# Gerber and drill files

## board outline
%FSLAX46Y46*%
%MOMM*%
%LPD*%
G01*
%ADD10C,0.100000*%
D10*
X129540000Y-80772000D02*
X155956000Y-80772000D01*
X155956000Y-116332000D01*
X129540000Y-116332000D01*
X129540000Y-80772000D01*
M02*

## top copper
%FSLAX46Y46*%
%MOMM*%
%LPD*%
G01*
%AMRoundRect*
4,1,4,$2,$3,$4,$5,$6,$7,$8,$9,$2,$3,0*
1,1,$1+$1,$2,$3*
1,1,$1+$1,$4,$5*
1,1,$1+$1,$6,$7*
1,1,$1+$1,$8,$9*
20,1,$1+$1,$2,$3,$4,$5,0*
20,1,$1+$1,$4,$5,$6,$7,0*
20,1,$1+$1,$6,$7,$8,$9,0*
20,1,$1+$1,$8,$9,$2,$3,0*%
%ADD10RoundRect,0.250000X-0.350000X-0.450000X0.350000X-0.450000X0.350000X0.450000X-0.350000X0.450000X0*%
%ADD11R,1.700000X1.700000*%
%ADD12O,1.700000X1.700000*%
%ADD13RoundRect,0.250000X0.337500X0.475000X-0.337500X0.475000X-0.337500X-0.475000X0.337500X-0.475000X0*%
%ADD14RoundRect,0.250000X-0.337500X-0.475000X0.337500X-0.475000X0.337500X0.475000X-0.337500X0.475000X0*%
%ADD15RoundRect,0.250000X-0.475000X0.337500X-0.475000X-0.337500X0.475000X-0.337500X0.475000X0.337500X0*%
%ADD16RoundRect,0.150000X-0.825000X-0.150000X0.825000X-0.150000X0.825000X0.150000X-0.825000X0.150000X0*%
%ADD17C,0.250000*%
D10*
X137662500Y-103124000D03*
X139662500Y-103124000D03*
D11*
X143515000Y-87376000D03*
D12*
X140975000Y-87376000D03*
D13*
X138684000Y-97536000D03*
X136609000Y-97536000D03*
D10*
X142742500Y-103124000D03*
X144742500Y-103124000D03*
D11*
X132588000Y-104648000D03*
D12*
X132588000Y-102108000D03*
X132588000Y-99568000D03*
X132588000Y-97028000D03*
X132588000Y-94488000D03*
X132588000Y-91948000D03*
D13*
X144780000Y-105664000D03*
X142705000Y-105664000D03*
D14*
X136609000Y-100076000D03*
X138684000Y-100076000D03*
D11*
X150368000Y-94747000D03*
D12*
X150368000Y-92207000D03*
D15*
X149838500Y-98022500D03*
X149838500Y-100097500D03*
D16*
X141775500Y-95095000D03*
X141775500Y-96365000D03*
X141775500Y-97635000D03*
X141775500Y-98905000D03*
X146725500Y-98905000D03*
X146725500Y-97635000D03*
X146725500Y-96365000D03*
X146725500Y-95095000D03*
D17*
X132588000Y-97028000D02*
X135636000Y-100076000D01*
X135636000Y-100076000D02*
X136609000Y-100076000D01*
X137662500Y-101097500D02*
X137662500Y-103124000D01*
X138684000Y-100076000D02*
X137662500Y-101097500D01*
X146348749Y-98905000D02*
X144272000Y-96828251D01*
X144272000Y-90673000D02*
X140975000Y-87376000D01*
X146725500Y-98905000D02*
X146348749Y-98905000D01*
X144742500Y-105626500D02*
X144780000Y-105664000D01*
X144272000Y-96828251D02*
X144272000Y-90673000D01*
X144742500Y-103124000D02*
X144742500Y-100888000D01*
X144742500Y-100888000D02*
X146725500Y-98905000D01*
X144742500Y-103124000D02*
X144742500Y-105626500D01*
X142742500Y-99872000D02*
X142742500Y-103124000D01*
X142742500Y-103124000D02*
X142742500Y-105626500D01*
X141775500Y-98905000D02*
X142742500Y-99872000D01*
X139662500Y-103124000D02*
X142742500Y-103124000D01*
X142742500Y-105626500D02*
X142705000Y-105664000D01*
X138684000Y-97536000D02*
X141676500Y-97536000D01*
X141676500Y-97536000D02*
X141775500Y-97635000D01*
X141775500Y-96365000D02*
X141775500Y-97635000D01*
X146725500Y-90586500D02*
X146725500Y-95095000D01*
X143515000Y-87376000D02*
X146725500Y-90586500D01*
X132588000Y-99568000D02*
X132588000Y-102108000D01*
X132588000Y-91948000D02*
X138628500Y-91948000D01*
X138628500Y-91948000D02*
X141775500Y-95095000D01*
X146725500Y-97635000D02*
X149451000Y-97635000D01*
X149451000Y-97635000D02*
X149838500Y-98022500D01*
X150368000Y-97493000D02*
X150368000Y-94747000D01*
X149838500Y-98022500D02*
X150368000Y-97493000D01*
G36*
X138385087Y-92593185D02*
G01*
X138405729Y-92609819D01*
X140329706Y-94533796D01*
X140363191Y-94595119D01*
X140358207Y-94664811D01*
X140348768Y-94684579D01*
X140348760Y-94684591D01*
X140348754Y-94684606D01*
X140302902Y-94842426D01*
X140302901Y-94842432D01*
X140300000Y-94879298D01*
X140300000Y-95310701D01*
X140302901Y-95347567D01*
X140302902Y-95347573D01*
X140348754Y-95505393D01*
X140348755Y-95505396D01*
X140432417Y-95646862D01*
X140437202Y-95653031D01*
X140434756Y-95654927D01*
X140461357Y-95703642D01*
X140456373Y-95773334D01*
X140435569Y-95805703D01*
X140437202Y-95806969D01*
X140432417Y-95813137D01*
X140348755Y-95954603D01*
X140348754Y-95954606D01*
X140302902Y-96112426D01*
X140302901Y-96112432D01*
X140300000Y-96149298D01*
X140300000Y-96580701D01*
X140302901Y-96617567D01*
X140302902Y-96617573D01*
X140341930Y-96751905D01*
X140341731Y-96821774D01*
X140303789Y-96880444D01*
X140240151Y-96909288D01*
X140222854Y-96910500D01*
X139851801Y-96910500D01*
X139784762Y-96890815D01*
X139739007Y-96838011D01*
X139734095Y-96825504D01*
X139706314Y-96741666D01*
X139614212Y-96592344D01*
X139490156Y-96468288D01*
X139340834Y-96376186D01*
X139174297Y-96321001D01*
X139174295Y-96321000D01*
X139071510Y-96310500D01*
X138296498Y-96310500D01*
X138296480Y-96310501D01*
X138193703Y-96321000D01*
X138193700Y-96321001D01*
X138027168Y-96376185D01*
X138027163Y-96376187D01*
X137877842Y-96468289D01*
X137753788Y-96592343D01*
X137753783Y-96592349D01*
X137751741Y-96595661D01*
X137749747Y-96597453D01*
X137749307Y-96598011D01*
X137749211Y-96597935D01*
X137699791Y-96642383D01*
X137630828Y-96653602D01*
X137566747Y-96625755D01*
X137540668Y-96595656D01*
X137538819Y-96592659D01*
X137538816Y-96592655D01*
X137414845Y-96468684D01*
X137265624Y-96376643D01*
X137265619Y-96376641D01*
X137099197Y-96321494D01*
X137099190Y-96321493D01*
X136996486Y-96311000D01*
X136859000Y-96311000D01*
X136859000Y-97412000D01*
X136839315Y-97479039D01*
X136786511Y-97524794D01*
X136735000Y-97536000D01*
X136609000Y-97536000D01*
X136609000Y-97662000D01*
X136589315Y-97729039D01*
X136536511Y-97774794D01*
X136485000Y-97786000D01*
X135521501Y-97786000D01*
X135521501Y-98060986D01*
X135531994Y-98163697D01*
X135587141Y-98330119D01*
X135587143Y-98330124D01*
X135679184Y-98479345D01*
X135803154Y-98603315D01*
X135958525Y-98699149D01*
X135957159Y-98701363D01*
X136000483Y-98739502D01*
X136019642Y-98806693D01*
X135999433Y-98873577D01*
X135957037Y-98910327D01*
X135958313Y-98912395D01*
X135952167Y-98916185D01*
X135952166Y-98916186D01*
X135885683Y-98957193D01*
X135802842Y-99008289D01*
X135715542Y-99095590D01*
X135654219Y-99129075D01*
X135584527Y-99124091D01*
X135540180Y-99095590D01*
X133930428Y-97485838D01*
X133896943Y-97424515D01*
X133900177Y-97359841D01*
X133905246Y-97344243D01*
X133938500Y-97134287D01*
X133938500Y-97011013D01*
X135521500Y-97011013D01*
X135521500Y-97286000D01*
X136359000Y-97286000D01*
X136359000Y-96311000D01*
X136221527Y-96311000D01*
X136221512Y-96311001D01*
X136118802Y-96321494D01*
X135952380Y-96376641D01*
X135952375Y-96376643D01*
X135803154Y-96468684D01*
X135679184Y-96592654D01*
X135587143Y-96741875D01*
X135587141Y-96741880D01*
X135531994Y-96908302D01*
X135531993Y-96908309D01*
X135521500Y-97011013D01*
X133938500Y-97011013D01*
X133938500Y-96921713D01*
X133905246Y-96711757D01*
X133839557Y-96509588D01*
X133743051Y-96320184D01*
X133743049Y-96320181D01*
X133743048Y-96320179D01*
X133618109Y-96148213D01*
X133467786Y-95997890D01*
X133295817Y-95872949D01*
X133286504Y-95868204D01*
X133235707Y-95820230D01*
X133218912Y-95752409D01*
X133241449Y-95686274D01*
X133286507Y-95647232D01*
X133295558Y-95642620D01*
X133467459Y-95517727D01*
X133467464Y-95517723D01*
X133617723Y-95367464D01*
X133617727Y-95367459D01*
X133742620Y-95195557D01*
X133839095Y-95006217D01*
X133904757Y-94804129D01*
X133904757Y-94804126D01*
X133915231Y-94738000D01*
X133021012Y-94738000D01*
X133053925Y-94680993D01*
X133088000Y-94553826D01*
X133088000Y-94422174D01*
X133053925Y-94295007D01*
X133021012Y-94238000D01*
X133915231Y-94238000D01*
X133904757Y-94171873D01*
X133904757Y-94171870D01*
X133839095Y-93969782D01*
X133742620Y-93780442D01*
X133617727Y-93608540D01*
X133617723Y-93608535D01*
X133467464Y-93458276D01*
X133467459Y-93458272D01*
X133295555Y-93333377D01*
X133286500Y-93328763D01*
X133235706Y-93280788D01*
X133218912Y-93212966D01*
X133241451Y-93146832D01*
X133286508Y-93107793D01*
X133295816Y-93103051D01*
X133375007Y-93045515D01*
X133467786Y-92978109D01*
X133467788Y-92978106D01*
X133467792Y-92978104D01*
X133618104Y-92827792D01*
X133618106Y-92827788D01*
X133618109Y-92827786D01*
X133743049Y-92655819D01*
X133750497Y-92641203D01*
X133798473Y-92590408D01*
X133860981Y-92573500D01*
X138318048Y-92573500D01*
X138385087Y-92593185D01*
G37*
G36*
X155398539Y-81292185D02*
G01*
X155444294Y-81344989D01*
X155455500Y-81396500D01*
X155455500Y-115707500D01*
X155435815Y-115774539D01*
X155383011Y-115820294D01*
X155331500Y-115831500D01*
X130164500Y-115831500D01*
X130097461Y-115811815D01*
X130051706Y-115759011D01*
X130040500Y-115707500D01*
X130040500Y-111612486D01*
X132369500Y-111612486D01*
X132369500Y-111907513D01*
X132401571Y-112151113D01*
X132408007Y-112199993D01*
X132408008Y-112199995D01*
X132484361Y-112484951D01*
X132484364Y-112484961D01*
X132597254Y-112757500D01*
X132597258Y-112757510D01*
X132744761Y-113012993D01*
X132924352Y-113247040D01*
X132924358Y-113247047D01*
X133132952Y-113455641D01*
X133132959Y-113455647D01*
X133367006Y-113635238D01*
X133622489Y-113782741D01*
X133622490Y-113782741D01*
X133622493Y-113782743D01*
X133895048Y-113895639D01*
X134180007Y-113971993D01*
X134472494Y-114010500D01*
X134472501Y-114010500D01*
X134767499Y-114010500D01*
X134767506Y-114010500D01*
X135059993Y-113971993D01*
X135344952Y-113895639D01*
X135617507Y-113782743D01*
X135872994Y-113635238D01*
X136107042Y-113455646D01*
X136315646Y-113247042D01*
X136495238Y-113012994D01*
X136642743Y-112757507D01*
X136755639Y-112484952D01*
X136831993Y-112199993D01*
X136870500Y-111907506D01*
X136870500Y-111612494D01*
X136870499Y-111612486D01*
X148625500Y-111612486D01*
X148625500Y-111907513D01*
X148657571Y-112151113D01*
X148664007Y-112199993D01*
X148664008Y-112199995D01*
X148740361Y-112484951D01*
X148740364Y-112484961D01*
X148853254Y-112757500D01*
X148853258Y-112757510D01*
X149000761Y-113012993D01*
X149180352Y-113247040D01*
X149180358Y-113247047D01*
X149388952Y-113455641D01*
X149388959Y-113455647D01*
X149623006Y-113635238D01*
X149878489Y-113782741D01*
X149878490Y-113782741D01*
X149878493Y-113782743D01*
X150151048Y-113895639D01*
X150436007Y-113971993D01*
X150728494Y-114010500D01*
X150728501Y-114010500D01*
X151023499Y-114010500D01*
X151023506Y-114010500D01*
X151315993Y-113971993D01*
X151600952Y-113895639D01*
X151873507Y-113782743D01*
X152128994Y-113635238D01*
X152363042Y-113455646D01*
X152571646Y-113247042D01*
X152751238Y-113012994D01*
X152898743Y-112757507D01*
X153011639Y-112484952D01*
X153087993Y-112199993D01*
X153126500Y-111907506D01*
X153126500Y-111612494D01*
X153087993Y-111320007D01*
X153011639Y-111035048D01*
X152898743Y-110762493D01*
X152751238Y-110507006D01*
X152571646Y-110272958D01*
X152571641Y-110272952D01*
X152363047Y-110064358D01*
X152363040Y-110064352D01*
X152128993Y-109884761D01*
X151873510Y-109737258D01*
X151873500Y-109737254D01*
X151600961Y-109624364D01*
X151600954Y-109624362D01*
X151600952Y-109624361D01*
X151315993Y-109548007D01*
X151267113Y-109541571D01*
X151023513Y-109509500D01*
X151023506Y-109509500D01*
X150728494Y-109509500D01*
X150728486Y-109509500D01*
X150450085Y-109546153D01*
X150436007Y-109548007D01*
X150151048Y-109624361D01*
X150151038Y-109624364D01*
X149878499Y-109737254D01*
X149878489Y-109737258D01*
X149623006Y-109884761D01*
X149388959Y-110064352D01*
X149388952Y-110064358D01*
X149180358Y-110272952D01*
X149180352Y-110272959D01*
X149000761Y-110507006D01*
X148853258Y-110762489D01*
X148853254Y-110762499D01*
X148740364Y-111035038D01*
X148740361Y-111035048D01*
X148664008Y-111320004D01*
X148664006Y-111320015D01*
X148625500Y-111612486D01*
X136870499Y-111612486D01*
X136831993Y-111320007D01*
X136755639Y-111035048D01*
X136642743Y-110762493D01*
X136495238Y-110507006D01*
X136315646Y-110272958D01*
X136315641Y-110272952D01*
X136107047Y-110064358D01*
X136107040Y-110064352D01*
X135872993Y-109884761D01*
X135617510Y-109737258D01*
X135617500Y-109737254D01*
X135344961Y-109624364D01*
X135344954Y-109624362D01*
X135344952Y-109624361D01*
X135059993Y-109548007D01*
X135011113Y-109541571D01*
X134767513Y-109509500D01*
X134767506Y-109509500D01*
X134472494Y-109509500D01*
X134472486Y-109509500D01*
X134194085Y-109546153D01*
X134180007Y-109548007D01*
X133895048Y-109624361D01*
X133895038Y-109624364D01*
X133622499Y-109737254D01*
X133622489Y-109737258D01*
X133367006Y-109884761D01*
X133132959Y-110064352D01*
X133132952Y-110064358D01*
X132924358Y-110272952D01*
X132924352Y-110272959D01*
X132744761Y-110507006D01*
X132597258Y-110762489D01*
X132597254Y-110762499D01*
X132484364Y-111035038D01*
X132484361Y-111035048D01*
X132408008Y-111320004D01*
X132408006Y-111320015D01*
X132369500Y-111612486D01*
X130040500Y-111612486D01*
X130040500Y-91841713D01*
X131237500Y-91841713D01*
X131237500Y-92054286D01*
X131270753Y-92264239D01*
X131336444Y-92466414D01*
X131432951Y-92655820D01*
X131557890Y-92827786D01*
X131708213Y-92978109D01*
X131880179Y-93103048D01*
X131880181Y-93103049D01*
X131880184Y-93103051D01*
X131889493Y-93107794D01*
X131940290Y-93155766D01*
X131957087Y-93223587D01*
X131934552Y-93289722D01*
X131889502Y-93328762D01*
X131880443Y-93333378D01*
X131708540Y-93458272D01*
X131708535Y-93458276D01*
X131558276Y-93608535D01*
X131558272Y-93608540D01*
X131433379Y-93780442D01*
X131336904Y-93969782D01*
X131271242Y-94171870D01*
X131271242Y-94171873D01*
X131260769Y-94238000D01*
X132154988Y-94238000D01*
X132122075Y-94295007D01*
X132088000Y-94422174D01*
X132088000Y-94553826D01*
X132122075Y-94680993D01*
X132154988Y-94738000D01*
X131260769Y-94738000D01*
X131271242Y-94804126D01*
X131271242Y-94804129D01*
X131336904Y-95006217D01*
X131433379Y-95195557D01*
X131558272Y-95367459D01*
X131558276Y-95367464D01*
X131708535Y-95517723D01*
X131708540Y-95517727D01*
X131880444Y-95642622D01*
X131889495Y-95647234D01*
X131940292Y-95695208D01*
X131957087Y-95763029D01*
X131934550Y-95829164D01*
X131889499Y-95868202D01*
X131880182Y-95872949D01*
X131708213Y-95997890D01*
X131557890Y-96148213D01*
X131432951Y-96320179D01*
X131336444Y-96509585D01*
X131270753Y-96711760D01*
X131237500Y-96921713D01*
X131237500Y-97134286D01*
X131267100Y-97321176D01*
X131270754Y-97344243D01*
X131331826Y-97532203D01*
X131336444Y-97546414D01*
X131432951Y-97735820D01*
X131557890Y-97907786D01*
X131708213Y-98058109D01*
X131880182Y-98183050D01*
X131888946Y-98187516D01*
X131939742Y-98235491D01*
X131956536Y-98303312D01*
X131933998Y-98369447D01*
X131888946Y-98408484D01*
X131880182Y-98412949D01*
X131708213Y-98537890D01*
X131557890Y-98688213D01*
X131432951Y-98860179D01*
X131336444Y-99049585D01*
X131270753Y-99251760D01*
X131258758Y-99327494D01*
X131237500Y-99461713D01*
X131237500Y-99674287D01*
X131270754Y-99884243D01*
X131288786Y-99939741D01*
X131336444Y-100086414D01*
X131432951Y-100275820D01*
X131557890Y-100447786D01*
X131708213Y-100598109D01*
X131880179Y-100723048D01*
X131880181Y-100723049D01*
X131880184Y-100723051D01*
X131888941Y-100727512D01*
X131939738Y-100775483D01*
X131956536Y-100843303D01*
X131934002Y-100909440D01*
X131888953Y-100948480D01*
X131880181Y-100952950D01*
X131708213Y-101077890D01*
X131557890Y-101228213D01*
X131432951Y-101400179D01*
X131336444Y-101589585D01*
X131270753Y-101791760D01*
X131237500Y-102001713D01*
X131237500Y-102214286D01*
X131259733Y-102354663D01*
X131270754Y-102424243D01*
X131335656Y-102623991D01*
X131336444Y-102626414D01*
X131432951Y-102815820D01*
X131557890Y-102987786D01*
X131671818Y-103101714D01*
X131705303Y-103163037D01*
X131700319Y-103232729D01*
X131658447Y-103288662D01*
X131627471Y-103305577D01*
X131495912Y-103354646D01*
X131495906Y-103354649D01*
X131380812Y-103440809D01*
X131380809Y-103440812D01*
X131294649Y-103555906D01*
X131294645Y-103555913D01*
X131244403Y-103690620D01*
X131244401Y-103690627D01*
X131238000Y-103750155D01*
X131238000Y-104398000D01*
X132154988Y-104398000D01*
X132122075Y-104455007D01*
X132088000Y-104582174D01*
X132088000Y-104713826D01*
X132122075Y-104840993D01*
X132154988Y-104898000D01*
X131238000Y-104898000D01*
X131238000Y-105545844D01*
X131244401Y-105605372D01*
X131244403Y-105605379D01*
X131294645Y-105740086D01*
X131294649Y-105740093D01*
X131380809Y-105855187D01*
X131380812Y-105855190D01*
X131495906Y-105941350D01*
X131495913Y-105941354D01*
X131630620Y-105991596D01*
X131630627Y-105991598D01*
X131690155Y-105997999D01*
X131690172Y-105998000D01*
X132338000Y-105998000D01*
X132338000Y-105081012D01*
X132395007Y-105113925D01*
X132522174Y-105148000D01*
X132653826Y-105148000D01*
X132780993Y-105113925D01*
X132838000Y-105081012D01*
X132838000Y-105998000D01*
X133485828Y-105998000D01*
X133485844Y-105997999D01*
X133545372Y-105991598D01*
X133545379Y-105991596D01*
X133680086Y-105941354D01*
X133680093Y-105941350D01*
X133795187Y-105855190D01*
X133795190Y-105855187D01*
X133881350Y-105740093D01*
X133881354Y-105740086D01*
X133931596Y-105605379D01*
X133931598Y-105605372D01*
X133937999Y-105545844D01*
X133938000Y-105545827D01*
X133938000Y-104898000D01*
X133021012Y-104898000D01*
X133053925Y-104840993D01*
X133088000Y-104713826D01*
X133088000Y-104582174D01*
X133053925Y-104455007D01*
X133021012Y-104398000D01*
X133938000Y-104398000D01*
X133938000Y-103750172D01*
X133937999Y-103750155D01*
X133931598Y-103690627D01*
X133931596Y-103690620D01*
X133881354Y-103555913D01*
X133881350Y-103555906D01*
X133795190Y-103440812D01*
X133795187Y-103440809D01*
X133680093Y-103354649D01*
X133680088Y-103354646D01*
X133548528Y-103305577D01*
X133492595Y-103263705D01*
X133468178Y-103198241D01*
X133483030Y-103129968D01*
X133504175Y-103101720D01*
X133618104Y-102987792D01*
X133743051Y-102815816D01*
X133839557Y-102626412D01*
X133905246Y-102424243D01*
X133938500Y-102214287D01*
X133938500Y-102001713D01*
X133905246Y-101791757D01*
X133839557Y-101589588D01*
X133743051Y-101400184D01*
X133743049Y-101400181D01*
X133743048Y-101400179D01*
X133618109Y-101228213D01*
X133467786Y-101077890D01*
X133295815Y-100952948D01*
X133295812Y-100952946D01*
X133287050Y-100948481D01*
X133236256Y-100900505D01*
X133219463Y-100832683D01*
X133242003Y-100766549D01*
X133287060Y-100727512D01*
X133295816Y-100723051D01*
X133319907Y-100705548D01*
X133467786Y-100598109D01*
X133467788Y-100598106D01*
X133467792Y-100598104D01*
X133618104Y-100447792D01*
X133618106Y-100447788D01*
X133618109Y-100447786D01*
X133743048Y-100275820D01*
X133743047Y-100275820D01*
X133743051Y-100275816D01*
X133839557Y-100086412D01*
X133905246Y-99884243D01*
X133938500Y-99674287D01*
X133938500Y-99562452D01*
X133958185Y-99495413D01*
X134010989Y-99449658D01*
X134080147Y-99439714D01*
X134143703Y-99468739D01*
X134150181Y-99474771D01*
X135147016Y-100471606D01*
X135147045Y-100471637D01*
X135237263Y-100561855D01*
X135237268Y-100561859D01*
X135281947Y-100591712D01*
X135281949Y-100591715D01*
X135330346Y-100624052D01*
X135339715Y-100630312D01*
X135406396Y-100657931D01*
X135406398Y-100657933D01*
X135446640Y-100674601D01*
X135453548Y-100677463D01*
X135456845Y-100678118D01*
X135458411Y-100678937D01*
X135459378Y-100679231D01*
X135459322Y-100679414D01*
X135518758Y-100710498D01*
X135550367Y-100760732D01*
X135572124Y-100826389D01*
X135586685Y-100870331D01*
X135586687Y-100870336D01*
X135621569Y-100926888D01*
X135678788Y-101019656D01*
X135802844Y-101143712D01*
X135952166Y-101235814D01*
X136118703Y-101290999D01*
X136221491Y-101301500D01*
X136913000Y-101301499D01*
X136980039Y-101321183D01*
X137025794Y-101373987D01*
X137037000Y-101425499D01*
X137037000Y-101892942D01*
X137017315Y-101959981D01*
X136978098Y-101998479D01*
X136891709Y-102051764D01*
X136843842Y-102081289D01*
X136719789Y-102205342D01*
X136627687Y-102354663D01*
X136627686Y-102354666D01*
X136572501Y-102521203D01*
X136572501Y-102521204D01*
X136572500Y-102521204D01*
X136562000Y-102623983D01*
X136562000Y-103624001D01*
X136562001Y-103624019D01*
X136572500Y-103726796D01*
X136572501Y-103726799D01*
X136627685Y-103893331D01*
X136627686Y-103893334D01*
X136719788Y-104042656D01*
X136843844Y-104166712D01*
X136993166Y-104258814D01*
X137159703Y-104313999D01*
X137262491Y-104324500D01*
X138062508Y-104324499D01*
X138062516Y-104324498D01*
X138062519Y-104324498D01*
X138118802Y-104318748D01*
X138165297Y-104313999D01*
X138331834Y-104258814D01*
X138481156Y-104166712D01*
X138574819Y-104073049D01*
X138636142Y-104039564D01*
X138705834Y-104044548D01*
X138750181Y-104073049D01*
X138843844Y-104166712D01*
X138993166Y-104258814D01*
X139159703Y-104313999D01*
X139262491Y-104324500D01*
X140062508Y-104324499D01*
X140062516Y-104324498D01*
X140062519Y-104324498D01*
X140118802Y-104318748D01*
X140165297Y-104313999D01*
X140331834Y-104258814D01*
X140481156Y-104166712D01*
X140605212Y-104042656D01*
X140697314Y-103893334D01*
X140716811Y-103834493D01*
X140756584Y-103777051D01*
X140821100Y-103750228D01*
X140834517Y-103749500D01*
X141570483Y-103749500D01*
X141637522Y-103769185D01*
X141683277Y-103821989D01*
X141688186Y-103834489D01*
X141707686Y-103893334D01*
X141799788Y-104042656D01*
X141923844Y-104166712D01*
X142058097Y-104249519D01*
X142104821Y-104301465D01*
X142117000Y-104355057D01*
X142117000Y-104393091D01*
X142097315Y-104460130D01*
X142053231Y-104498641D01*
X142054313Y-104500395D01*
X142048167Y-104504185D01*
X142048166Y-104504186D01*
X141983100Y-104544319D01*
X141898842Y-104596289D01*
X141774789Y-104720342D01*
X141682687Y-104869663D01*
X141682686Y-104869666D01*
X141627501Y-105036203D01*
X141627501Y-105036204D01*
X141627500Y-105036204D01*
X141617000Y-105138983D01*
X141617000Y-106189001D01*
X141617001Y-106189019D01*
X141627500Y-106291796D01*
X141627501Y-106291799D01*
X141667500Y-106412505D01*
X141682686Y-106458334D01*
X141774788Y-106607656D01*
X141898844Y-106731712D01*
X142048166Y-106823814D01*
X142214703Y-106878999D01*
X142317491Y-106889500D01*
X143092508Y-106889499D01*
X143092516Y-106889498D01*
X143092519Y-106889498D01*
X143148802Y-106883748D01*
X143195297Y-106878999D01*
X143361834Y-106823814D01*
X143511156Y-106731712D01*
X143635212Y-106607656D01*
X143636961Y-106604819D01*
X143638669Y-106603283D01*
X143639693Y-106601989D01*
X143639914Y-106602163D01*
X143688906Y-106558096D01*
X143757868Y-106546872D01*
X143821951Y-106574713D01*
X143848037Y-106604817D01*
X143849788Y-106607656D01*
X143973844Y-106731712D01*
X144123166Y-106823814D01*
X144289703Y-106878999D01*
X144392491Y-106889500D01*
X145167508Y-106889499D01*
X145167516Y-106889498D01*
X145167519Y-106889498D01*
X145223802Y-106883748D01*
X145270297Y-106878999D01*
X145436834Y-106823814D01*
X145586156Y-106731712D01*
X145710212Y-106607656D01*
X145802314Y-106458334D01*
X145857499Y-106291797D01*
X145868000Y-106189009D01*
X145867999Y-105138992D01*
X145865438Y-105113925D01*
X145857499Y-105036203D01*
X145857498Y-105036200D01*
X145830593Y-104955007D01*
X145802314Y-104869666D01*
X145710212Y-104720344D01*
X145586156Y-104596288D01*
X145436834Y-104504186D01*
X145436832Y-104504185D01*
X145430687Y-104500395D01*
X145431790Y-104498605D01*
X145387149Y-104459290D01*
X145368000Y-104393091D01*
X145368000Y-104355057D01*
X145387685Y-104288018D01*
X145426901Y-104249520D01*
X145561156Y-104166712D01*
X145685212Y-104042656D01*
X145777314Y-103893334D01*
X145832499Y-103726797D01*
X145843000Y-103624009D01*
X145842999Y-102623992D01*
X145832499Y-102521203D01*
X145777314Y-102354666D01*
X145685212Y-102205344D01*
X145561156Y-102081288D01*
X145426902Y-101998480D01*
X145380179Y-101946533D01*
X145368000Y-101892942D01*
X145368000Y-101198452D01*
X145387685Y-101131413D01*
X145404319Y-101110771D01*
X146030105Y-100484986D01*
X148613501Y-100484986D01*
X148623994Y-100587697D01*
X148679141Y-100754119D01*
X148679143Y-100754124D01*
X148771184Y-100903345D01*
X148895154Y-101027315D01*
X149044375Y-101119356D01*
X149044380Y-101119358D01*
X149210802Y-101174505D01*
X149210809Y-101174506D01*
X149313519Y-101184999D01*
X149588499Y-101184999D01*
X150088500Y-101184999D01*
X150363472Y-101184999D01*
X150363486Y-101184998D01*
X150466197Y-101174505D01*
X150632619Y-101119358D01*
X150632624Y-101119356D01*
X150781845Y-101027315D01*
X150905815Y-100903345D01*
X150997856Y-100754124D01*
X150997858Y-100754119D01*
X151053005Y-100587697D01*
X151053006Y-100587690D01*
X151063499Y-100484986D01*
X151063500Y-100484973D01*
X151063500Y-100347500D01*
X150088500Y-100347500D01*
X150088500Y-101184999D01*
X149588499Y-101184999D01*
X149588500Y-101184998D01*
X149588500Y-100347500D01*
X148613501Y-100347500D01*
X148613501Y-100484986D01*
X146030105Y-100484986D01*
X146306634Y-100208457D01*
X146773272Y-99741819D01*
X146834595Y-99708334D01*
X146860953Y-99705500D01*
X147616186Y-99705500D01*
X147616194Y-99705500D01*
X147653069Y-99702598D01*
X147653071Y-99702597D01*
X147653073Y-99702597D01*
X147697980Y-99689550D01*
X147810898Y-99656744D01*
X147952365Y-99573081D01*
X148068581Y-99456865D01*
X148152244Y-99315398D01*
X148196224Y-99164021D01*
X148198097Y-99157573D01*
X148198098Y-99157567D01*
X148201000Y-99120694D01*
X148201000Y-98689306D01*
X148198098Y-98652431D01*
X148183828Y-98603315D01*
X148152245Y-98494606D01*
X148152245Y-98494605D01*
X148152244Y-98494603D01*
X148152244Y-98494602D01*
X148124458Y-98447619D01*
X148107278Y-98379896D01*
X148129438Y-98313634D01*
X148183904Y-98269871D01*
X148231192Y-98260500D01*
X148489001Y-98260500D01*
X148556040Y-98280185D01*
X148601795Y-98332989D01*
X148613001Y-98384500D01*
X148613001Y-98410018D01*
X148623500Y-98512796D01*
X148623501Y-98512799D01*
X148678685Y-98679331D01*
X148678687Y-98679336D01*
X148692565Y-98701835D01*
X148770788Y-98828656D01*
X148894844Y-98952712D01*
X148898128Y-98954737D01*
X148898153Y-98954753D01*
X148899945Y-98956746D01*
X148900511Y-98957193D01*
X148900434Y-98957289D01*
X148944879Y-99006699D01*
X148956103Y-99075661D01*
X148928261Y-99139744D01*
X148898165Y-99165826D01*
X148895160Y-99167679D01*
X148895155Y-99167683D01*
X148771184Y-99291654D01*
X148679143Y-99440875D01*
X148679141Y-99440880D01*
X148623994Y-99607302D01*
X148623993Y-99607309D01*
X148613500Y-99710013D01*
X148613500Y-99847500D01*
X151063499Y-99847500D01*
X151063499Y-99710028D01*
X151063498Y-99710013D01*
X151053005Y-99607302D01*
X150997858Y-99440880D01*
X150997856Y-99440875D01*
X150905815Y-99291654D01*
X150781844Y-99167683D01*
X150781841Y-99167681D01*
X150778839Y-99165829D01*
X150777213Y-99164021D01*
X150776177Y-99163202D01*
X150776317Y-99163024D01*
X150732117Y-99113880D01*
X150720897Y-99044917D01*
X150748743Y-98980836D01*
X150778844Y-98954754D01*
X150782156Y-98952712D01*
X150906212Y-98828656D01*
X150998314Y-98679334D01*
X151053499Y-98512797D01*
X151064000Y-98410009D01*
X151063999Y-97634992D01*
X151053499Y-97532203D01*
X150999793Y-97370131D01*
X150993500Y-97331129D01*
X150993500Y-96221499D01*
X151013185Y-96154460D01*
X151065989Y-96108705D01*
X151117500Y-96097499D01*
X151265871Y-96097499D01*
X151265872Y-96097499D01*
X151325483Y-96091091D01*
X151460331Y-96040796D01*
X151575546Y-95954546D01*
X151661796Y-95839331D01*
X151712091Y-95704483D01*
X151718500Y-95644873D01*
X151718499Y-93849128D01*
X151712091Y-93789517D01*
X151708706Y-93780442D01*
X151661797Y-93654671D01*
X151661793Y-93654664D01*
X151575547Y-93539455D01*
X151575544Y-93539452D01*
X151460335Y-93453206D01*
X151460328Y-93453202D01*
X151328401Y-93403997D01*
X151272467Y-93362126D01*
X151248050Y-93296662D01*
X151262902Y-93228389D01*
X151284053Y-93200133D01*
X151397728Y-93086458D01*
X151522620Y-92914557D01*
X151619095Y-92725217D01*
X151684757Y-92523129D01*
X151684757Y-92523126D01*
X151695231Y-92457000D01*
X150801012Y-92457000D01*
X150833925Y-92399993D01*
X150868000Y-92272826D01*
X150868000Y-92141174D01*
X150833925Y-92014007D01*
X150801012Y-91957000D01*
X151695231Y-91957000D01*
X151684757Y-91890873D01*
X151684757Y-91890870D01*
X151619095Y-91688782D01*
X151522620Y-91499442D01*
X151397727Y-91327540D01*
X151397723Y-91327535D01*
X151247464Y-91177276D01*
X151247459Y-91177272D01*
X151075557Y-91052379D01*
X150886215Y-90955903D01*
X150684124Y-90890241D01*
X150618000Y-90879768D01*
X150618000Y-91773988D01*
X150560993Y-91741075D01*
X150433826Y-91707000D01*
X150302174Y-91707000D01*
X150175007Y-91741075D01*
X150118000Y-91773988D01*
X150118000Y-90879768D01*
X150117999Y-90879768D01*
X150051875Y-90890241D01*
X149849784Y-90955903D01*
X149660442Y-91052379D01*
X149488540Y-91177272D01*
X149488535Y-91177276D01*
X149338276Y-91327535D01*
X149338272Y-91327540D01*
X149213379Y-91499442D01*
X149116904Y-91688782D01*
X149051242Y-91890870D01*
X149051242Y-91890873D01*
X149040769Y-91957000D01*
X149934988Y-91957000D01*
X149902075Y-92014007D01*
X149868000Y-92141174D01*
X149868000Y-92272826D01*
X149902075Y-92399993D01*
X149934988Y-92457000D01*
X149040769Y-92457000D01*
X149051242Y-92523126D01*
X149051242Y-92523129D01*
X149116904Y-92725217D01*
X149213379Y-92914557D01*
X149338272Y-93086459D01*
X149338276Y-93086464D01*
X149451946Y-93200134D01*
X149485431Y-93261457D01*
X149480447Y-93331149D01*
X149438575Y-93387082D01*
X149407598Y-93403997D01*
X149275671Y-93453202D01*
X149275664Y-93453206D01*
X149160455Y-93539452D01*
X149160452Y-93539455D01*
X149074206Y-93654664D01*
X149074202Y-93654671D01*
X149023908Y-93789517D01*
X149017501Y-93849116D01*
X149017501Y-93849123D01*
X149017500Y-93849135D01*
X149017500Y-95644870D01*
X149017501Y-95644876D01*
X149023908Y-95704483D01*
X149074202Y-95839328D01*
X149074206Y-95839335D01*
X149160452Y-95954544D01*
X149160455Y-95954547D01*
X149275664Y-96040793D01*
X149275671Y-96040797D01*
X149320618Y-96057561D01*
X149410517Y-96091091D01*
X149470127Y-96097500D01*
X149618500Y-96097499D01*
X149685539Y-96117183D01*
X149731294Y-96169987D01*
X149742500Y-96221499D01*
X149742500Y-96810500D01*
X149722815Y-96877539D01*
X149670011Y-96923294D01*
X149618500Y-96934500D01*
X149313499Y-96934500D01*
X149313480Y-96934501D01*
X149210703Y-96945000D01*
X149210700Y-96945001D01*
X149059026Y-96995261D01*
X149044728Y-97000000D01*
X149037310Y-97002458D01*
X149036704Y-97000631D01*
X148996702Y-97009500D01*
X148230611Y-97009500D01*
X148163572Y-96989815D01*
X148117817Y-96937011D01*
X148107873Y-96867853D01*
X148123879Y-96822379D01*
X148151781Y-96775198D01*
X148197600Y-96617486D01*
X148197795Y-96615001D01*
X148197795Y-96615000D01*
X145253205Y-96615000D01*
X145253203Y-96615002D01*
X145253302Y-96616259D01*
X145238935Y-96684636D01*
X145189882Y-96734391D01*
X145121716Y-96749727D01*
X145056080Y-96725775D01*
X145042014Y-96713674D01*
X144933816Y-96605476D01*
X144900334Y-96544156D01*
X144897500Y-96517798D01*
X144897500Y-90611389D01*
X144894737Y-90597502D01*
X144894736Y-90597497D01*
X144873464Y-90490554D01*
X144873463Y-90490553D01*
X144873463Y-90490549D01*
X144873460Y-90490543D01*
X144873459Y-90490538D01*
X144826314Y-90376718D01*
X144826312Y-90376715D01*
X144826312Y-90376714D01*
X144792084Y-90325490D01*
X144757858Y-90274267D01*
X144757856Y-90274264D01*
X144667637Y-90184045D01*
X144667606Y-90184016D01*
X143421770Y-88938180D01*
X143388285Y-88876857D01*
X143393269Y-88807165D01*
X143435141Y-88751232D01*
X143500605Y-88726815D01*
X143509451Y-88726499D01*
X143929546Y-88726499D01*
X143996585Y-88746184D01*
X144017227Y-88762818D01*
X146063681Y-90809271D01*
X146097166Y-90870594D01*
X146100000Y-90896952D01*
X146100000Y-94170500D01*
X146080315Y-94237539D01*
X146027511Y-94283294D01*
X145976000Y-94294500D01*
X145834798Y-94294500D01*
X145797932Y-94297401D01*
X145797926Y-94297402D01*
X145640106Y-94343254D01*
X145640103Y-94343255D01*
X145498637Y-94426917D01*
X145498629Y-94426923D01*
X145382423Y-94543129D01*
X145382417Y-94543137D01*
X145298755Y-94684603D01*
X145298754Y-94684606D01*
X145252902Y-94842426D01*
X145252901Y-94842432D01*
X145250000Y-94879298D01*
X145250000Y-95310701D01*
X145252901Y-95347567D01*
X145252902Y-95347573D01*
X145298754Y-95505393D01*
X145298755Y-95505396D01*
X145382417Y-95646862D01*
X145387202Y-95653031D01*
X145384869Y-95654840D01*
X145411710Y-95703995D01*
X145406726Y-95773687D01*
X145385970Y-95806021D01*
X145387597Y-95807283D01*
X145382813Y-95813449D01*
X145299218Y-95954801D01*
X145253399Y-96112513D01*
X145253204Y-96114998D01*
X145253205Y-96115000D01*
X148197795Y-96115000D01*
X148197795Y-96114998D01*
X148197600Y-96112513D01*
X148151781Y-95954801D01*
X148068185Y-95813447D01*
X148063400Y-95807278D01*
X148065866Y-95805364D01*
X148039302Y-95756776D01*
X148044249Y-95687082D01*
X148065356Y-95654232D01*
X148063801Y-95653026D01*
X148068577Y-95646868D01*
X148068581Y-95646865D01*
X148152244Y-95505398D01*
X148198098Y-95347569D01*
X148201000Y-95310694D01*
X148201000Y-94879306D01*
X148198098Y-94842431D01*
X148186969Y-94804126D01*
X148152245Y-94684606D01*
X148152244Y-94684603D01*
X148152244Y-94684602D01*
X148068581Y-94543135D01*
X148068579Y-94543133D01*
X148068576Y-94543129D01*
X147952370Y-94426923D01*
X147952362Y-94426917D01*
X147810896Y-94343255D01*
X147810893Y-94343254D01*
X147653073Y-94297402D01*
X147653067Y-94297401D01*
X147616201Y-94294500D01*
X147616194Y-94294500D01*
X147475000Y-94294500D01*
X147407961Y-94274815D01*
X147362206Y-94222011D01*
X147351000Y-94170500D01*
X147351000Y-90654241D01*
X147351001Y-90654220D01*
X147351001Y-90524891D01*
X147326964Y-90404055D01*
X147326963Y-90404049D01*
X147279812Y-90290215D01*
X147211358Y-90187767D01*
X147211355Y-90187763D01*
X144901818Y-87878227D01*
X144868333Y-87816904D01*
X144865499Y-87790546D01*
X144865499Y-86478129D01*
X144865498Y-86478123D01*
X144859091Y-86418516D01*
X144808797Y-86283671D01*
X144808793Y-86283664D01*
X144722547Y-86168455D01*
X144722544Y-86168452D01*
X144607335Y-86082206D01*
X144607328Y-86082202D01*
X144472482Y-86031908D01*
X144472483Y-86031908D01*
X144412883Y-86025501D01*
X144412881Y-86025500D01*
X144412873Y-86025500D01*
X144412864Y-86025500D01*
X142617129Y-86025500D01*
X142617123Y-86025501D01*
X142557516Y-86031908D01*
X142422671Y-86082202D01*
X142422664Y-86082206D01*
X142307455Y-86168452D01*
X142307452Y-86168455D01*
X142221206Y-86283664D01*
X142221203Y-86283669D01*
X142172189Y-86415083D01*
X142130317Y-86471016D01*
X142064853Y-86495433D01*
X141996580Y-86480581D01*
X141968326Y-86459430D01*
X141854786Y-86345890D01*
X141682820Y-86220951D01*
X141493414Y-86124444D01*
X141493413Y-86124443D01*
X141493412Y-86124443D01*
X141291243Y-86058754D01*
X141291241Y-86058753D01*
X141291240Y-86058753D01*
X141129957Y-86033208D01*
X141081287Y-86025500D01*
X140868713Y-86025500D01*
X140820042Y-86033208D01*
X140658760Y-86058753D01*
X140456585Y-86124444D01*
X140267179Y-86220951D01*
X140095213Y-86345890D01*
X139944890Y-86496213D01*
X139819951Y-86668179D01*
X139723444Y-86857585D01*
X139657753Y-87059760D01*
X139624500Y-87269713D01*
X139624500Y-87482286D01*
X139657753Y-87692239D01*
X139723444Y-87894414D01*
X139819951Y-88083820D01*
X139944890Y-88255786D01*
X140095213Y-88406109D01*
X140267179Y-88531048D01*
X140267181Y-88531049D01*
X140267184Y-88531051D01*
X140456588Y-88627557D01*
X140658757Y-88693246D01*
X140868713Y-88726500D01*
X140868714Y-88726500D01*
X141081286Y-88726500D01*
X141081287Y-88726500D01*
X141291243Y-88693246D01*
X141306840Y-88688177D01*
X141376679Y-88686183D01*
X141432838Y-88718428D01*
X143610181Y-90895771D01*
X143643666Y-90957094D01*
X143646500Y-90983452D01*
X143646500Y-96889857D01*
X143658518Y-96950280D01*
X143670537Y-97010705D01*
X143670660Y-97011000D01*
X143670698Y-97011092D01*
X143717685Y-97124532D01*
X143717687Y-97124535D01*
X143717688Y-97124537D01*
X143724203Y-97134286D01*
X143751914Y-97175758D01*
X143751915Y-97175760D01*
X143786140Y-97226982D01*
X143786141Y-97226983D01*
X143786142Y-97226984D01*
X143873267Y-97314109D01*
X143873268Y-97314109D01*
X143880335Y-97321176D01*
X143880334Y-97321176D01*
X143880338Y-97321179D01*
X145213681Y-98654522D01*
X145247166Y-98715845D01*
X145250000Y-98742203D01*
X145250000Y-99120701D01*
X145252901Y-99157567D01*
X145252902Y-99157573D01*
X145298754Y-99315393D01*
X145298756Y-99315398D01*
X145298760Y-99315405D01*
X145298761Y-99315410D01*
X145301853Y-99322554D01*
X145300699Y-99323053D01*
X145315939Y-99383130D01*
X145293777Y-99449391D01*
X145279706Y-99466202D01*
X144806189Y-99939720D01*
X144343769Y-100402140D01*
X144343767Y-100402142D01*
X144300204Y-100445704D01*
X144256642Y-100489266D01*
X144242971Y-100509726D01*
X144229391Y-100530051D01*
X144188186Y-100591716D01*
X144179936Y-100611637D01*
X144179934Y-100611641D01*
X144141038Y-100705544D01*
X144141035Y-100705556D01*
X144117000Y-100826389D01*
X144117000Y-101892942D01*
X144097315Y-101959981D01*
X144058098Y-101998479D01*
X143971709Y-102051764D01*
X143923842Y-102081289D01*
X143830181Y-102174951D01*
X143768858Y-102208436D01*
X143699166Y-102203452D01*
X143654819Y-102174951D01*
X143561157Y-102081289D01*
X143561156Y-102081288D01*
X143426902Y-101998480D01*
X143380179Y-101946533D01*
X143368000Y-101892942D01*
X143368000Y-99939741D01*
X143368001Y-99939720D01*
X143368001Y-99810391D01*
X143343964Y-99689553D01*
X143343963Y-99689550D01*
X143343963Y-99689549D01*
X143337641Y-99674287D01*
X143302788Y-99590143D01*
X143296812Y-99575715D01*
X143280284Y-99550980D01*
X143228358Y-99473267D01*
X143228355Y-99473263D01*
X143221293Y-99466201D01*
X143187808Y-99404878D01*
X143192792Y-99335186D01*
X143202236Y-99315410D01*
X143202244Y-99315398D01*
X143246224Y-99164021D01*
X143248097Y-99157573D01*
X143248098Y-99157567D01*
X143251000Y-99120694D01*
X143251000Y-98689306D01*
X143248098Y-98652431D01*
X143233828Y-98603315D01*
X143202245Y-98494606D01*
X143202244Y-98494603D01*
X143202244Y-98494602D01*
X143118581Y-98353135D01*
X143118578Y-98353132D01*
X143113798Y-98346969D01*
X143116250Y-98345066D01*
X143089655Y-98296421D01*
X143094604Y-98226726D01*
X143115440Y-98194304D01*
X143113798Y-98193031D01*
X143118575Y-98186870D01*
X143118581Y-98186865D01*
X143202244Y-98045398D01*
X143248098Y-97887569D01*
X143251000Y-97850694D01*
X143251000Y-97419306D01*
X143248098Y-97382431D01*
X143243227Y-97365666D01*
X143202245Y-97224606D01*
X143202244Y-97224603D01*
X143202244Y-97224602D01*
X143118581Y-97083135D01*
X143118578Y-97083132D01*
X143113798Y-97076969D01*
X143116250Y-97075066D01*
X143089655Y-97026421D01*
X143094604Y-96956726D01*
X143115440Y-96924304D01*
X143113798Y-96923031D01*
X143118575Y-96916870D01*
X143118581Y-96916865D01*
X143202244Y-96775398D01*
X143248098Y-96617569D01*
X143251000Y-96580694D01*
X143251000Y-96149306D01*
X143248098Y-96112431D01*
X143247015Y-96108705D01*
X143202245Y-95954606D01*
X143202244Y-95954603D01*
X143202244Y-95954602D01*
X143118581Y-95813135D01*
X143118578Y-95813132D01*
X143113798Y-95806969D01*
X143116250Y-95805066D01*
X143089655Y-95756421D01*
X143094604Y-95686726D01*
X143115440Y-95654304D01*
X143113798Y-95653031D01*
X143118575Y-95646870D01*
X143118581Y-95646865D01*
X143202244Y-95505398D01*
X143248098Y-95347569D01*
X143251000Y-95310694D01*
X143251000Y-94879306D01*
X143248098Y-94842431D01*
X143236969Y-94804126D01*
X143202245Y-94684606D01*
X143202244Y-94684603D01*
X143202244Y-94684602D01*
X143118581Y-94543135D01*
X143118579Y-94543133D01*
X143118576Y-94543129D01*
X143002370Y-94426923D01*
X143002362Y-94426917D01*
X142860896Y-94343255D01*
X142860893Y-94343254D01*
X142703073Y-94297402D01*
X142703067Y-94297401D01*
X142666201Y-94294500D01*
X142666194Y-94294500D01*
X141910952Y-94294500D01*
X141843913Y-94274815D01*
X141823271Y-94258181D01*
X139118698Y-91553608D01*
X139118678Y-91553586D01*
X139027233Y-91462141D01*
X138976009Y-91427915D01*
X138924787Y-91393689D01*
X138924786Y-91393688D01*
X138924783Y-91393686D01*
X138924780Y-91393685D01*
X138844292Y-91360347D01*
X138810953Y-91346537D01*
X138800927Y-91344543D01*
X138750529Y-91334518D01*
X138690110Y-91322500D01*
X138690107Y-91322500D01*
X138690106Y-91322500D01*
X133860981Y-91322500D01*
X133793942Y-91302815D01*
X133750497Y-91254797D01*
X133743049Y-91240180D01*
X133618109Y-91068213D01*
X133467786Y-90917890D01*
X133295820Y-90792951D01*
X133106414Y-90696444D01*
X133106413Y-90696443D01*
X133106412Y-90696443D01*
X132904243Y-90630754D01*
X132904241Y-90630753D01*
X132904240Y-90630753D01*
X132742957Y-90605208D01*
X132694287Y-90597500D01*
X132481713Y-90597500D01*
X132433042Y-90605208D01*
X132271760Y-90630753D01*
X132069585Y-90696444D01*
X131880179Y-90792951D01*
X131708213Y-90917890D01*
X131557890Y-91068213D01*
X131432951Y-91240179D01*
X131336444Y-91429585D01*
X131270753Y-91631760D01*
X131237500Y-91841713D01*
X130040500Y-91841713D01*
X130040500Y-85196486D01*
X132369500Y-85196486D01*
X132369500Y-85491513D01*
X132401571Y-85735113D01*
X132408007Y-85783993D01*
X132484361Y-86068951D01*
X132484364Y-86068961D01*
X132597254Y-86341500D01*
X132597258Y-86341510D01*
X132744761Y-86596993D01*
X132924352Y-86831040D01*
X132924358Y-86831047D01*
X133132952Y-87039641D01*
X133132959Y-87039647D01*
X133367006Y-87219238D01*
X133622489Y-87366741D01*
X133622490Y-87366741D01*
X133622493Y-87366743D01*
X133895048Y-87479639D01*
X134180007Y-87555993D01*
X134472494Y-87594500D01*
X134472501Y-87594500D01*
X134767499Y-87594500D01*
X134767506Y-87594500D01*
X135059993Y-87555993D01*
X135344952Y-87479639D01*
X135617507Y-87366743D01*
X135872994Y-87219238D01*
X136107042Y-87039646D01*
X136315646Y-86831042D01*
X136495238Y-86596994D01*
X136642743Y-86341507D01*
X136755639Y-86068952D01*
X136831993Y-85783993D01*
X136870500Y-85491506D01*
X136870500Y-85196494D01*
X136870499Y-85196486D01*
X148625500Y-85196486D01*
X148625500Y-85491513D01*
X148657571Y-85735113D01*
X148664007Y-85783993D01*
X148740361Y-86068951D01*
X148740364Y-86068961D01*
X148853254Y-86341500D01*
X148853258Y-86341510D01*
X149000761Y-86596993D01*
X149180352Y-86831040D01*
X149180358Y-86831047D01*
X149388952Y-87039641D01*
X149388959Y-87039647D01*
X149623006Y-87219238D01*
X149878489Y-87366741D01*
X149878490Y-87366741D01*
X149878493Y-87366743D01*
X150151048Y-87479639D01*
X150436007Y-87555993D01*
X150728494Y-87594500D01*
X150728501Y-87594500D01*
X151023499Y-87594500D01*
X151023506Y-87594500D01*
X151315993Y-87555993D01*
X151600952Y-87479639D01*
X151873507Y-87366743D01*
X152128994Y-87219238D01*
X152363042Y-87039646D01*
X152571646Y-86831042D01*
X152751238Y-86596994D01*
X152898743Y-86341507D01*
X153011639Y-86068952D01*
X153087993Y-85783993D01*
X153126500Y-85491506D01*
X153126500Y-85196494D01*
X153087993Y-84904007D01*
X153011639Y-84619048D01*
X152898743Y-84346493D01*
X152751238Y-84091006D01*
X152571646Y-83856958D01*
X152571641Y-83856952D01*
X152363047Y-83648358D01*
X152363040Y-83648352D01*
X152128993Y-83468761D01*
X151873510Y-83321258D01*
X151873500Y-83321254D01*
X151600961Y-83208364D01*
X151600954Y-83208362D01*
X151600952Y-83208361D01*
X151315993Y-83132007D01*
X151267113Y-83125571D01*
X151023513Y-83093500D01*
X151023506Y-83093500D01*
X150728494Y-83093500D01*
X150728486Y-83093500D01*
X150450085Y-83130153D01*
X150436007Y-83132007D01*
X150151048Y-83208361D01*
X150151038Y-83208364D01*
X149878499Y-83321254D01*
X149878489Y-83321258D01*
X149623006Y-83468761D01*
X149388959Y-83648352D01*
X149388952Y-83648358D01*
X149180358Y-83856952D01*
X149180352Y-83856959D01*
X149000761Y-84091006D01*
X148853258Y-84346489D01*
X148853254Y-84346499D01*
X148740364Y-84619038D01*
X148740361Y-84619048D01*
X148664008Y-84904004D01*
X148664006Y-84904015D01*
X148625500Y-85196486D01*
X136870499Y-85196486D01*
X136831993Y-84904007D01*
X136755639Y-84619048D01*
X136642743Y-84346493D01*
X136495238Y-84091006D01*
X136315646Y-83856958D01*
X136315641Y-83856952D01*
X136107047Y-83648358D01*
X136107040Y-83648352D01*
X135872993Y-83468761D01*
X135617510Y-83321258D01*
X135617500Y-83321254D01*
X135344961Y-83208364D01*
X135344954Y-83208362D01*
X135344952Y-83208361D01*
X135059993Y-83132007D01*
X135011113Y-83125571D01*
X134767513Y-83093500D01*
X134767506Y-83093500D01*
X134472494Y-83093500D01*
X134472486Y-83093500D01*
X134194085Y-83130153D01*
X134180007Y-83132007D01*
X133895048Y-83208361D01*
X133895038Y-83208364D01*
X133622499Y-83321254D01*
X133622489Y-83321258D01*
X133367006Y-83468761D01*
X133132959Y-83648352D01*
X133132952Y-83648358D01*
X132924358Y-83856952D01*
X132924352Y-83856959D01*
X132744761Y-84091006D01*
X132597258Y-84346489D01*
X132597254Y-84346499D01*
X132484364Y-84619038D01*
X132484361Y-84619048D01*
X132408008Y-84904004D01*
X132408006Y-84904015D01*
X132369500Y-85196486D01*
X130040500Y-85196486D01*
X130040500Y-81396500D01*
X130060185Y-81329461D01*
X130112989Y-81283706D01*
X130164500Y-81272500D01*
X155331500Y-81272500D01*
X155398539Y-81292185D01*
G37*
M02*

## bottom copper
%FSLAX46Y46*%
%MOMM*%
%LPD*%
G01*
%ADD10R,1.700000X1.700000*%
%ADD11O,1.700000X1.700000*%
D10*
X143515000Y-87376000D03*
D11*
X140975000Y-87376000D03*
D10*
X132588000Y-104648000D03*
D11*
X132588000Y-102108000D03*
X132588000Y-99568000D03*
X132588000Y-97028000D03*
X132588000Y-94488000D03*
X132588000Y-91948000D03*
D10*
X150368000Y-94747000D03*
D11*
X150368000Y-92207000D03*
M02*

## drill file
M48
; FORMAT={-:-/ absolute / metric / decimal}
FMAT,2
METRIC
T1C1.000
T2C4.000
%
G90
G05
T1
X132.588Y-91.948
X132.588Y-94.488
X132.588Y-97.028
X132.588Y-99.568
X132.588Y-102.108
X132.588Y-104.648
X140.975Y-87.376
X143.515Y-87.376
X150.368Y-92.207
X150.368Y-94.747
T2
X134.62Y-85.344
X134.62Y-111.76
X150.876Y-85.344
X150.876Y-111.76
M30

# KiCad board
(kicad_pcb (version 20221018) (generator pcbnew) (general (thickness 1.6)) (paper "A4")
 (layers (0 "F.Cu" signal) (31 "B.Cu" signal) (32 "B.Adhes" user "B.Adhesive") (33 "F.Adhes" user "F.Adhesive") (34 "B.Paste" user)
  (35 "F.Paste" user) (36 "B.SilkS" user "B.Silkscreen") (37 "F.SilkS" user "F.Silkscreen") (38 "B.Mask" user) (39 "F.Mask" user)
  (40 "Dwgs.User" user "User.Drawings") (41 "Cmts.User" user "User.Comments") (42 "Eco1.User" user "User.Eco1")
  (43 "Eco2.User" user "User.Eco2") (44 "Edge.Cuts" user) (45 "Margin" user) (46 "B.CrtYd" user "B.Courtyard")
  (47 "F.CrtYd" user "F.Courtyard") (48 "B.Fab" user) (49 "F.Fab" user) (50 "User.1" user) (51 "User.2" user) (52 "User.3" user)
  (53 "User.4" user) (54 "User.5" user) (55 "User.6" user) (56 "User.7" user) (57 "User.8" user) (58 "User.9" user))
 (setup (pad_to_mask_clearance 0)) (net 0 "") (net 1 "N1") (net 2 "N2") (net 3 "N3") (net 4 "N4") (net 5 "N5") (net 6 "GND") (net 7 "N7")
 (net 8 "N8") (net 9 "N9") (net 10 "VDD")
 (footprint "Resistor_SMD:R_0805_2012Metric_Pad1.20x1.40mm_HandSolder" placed (layer "F.Cu") (at 138.6625 103.124)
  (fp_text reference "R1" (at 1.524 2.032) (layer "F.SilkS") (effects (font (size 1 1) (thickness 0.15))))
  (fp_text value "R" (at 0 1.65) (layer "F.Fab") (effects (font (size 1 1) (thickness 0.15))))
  (pad "1" smd roundrect (at -1 0) (size 1.2 1.4) (layers "F.Cu" "F.Paste" "F.Mask") (roundrect_rratio 0.208333) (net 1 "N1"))
  (pad "2" smd roundrect (at 1 0) (size 1.2 1.4) (layers "F.Cu" "F.Paste" "F.Mask") (roundrect_rratio 0.208333) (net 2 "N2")))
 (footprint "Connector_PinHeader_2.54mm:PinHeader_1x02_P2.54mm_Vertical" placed (layer "F.Cu") (at 143.515 87.376 -90)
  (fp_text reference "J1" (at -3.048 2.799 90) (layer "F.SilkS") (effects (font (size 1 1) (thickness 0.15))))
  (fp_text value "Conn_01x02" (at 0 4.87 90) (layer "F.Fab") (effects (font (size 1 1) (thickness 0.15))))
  (pad "1" thru_hole rect (at 0 0 270) (size 1.7 1.7) (drill 1) (layers "*.Cu" "*.Mask") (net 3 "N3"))
  (pad "2" thru_hole oval (at 0 2.54 270) (size 1.7 1.7) (drill 1) (layers "*.Cu" "*.Mask") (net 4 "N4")))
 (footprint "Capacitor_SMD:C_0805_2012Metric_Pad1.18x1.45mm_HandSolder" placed (layer "F.Cu") (at 137.6465 97.536 180)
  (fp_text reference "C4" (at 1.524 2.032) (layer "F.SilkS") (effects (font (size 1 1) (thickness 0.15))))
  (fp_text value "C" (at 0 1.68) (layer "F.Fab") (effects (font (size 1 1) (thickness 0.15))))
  (pad "1" smd roundrect (at -1.0375 0 180) (size 1.175 1.45) (layers "F.Cu" "F.Paste" "F.Mask") (roundrect_rratio 0.212766) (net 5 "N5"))
  (pad "2" smd roundrect (at 1.0375 0 180) (size 1.175 1.45) (layers "F.Cu" "F.Paste" "F.Mask") (roundrect_rratio 0.212766) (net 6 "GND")))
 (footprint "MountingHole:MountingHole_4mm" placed (layer "F.Cu") (at 134.62 85.344)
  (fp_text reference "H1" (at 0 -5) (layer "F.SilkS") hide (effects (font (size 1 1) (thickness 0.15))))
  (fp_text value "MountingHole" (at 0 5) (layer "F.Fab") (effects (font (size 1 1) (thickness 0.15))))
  (pad "" np_thru_hole circle (at 0 0) (size 4 4) (drill 4) (layers "*.Cu" "*.Mask")))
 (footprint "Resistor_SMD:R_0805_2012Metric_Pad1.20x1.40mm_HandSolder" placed (layer "F.Cu") (at 143.7425 103.124)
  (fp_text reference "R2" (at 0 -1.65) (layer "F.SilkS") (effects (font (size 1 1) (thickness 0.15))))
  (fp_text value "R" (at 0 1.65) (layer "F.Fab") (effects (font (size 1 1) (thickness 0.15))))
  (pad "1" smd roundrect (at -1 0) (size 1.2 1.4) (layers "F.Cu" "F.Paste" "F.Mask") (roundrect_rratio 0.208333) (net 2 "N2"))
  (pad "2" smd roundrect (at 1 0) (size 1.2 1.4) (layers "F.Cu" "F.Paste" "F.Mask") (roundrect_rratio 0.208333) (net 4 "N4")))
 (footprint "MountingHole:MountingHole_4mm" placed (layer "F.Cu") (at 134.62 111.76)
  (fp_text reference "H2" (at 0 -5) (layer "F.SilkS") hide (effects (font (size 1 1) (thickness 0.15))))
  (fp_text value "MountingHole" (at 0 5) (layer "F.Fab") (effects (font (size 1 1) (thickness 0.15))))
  (pad "" np_thru_hole circle (at 0 0) (size 4 4) (drill 4) (layers "*.Cu" "*.Mask")))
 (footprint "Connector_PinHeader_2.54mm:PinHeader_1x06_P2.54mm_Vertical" (layer "F.Cu") (at 132.588 104.648 180)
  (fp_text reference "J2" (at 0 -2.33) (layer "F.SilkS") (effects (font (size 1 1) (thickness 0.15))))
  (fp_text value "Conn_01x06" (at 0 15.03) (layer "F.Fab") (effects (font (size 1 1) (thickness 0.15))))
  (pad "1" thru_hole rect (at 0 0 180) (size 1.7 1.7) (drill 1) (layers "*.Cu" "*.Mask") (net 6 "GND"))
  (pad "2" thru_hole oval (at 0 2.54 180) (size 1.7 1.7) (drill 1) (layers "*.Cu" "*.Mask") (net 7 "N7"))
  (pad "3" thru_hole oval (at 0 5.08 180) (size 1.7 1.7) (drill 1) (layers "*.Cu" "*.Mask") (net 7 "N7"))
  (pad "4" thru_hole oval (at 0 7.62 180) (size 1.7 1.7) (drill 1) (layers "*.Cu" "*.Mask") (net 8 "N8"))
  (pad "5" thru_hole oval (at 0 10.16 180) (size 1.7 1.7) (drill 1) (layers "*.Cu" "*.Mask") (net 6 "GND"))
  (pad "6" thru_hole oval (at 0 12.7 180) (size 1.7 1.7) (drill 1) (layers "*.Cu" "*.Mask") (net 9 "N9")))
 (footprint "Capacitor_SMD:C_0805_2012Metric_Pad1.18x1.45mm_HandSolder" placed (layer "F.Cu") (at 143.7425 105.664 180)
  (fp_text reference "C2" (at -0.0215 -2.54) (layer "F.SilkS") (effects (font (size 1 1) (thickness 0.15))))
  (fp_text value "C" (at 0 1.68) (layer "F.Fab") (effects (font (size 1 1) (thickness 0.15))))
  (pad "1" smd roundrect (at -1.0375 0 180) (size 1.175 1.45) (layers "F.Cu" "F.Paste" "F.Mask") (roundrect_rratio 0.212766) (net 4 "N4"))
  (pad "2" smd roundrect (at 1.0375 0 180) (size 1.175 1.45) (layers "F.Cu" "F.Paste" "F.Mask") (roundrect_rratio 0.212766) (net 2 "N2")))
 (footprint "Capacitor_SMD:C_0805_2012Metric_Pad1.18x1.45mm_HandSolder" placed (layer "F.Cu") (at 137.6465 100.076)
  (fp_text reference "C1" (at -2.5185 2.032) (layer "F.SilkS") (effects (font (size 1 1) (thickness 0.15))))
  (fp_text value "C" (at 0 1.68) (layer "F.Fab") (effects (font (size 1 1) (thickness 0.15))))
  (pad "1" smd roundrect (at -1.0375 0) (size 1.175 1.45) (layers "F.Cu" "F.Paste" "F.Mask") (roundrect_rratio 0.212766) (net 8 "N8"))
  (pad "2" smd roundrect (at 1.0375 0) (size 1.175 1.45) (layers "F.Cu" "F.Paste" "F.Mask") (roundrect_rratio 0.212766) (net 1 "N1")))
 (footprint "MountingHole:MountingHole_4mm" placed (layer "F.Cu") (at 150.876 85.344)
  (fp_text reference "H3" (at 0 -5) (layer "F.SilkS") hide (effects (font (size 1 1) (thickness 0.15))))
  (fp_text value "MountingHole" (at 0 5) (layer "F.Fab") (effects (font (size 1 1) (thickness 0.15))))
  (pad "" np_thru_hole circle (at 0 0) (size 4 4) (drill 4) (layers "*.Cu" "*.Mask")))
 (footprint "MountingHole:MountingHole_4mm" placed (layer "F.Cu") (at 150.876 111.76)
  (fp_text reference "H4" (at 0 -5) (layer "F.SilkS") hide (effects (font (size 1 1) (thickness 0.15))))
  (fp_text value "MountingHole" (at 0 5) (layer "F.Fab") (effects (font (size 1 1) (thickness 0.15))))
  (pad "" np_thru_hole circle (at 0 0) (size 4 4) (drill 4) (layers "*.Cu" "*.Mask")))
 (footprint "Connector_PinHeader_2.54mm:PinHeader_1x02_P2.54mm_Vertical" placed (layer "F.Cu") (at 150.368 94.747 180)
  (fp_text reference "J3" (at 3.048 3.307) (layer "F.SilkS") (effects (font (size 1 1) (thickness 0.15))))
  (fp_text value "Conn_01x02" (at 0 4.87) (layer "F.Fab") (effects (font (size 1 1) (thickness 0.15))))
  (pad "1" thru_hole rect (at 0 0 180) (size 1.7 1.7) (drill 1) (layers "*.Cu" "*.Mask") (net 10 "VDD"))
  (pad "2" thru_hole oval (at 0 2.54 180) (size 1.7 1.7) (drill 1) (layers "*.Cu" "*.Mask") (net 6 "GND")))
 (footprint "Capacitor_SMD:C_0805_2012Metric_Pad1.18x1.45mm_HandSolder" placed (layer "F.Cu") (at 149.8385 99.06 -90)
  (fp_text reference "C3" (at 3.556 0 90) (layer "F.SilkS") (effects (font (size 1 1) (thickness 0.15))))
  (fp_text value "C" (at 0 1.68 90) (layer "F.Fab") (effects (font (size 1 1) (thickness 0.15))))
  (pad "1" smd roundrect (at -1.0375 0 270) (size 1.175 1.45) (layers "F.Cu" "F.Paste" "F.Mask") (roundrect_rratio 0.212766) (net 10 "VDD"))
  (pad "2" smd roundrect (at 1.0375 0 270) (size 1.175 1.45) (layers "F.Cu" "F.Paste" "F.Mask") (roundrect_rratio 0.212766) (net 6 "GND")))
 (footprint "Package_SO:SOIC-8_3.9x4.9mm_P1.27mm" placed (layer "F.Cu") (at 144.2505 97)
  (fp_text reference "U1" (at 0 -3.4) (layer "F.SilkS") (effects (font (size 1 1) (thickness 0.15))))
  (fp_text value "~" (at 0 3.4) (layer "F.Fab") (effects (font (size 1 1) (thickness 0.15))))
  (pad "1" smd roundrect (at -2.475 -1.905) (size 1.95 0.6) (layers "F.Cu" "F.Paste" "F.Mask") (roundrect_rratio 0.25) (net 9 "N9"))
  (pad "2" smd roundrect (at -2.475 -0.635) (size 1.95 0.6) (layers "F.Cu" "F.Paste" "F.Mask") (roundrect_rratio 0.25) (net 5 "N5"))
  (pad "3" smd roundrect (at -2.475 0.635) (size 1.95 0.6) (layers "F.Cu" "F.Paste" "F.Mask") (roundrect_rratio 0.25) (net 5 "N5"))
  (pad "4" smd roundrect (at -2.475 1.905) (size 1.95 0.6) (layers "F.Cu" "F.Paste" "F.Mask") (roundrect_rratio 0.25) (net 2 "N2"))
  (pad "5" smd roundrect (at 2.475 1.905) (size 1.95 0.6) (layers "F.Cu" "F.Paste" "F.Mask") (roundrect_rratio 0.25) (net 4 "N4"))
  (pad "6" smd roundrect (at 2.475 0.635) (size 1.95 0.6) (layers "F.Cu" "F.Paste" "F.Mask") (roundrect_rratio 0.25) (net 10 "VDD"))
  (pad "7" smd roundrect (at 2.475 -0.635) (size 1.95 0.6) (layers "F.Cu" "F.Paste" "F.Mask") (roundrect_rratio 0.25) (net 6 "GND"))
  (pad "8" smd roundrect (at 2.475 -1.905) (size 1.95 0.6) (layers "F.Cu" "F.Paste" "F.Mask") (roundrect_rratio 0.25) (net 3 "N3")))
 (gr_rect (start 129.54 80.772) (end 155.956 116.332) (stroke (width 0.1) (type default)) (fill none) (layer "Edge.Cuts"))
 (segment (start 132.588 97.028) (end 135.636 100.076) (width 0.25) (layer "F.Cu") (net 8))
 (segment (start 135.636 100.076) (end 136.609 100.076) (width 0.25) (layer "F.Cu") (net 8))
 (segment (start 137.6625 101.0975) (end 137.6625 103.124) (width 0.25) (layer "F.Cu") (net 1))
 (segment (start 138.684 100.076) (end 137.6625 101.0975) (width 0.25) (layer "F.Cu") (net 1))
 (segment (start 146.348749 98.905) (end 144.272 96.828251) (width 0.25) (layer "F.Cu") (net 4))
 (segment (start 144.272 90.673) (end 140.975 87.376) (width 0.25) (layer "F.Cu") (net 4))
 (segment (start 146.7255 98.905) (end 146.348749 98.905) (width 0.25) (layer "F.Cu") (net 4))
 (segment (start 144.7425 105.6265) (end 144.78 105.664) (width 0.25) (layer "F.Cu") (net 4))
 (segment (start 144.272 96.828251) (end 144.272 90.673) (width 0.25) (layer "F.Cu") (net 4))
 (segment (start 144.7425 103.124) (end 144.7425 100.888) (width 0.25) (layer "F.Cu") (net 4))
 (segment (start 144.7425 100.888) (end 146.7255 98.905) (width 0.25) (layer "F.Cu") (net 4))
 (segment (start 144.7425 103.124) (end 144.7425 105.6265) (width 0.25) (layer "F.Cu") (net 4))
 (segment (start 142.7425 99.872) (end 142.7425 103.124) (width 0.25) (layer "F.Cu") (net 2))
 (segment (start 142.7425 103.124) (end 142.7425 105.6265) (width 0.25) (layer "F.Cu") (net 2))
 (segment (start 141.7755 98.905) (end 142.7425 99.872) (width 0.25) (layer "F.Cu") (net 2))
 (segment (start 139.6625 103.124) (end 142.7425 103.124) (width 0.25) (layer "F.Cu") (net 2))
 (segment (start 142.7425 105.6265) (end 142.705 105.664) (width 0.25) (layer "F.Cu") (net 2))
 (segment (start 138.684 97.536) (end 141.6765 97.536) (width 0.25) (layer "F.Cu") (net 5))
 (segment (start 141.6765 97.536) (end 141.7755 97.635) (width 0.25) (layer "F.Cu") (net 5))
 (segment (start 141.7755 96.365) (end 141.7755 97.635) (width 0.25) (layer "F.Cu") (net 5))
 (segment (start 146.7255 90.5865) (end 146.7255 95.095) (width 0.25) (layer "F.Cu") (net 3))
 (segment (start 143.515 87.376) (end 146.7255 90.5865) (width 0.25) (layer "F.Cu") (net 3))
 (segment (start 132.588 99.568) (end 132.588 102.108) (width 0.25) (layer "F.Cu") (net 7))
 (segment (start 132.588 91.948) (end 138.6285 91.948) (width 0.25) (layer "F.Cu") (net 9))
 (segment (start 138.6285 91.948) (end 141.7755 95.095) (width 0.25) (layer "F.Cu") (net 9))
 (segment (start 146.7255 97.635) (end 149.451 97.635) (width 0.25) (layer "F.Cu") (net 10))
 (segment (start 149.451 97.635) (end 149.8385 98.0225) (width 0.25) (layer "F.Cu") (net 10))
 (segment (start 150.368 97.493) (end 150.368 94.747) (width 0.25) (layer "F.Cu") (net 10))
 (segment (start 149.8385 98.0225) (end 150.368 97.493) (width 0.25) (layer "F.Cu") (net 10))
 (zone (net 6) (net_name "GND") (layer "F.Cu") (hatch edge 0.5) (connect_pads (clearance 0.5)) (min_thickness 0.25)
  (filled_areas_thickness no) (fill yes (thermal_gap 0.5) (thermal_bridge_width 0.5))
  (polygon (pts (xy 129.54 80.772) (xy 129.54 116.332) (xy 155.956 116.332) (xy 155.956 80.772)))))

